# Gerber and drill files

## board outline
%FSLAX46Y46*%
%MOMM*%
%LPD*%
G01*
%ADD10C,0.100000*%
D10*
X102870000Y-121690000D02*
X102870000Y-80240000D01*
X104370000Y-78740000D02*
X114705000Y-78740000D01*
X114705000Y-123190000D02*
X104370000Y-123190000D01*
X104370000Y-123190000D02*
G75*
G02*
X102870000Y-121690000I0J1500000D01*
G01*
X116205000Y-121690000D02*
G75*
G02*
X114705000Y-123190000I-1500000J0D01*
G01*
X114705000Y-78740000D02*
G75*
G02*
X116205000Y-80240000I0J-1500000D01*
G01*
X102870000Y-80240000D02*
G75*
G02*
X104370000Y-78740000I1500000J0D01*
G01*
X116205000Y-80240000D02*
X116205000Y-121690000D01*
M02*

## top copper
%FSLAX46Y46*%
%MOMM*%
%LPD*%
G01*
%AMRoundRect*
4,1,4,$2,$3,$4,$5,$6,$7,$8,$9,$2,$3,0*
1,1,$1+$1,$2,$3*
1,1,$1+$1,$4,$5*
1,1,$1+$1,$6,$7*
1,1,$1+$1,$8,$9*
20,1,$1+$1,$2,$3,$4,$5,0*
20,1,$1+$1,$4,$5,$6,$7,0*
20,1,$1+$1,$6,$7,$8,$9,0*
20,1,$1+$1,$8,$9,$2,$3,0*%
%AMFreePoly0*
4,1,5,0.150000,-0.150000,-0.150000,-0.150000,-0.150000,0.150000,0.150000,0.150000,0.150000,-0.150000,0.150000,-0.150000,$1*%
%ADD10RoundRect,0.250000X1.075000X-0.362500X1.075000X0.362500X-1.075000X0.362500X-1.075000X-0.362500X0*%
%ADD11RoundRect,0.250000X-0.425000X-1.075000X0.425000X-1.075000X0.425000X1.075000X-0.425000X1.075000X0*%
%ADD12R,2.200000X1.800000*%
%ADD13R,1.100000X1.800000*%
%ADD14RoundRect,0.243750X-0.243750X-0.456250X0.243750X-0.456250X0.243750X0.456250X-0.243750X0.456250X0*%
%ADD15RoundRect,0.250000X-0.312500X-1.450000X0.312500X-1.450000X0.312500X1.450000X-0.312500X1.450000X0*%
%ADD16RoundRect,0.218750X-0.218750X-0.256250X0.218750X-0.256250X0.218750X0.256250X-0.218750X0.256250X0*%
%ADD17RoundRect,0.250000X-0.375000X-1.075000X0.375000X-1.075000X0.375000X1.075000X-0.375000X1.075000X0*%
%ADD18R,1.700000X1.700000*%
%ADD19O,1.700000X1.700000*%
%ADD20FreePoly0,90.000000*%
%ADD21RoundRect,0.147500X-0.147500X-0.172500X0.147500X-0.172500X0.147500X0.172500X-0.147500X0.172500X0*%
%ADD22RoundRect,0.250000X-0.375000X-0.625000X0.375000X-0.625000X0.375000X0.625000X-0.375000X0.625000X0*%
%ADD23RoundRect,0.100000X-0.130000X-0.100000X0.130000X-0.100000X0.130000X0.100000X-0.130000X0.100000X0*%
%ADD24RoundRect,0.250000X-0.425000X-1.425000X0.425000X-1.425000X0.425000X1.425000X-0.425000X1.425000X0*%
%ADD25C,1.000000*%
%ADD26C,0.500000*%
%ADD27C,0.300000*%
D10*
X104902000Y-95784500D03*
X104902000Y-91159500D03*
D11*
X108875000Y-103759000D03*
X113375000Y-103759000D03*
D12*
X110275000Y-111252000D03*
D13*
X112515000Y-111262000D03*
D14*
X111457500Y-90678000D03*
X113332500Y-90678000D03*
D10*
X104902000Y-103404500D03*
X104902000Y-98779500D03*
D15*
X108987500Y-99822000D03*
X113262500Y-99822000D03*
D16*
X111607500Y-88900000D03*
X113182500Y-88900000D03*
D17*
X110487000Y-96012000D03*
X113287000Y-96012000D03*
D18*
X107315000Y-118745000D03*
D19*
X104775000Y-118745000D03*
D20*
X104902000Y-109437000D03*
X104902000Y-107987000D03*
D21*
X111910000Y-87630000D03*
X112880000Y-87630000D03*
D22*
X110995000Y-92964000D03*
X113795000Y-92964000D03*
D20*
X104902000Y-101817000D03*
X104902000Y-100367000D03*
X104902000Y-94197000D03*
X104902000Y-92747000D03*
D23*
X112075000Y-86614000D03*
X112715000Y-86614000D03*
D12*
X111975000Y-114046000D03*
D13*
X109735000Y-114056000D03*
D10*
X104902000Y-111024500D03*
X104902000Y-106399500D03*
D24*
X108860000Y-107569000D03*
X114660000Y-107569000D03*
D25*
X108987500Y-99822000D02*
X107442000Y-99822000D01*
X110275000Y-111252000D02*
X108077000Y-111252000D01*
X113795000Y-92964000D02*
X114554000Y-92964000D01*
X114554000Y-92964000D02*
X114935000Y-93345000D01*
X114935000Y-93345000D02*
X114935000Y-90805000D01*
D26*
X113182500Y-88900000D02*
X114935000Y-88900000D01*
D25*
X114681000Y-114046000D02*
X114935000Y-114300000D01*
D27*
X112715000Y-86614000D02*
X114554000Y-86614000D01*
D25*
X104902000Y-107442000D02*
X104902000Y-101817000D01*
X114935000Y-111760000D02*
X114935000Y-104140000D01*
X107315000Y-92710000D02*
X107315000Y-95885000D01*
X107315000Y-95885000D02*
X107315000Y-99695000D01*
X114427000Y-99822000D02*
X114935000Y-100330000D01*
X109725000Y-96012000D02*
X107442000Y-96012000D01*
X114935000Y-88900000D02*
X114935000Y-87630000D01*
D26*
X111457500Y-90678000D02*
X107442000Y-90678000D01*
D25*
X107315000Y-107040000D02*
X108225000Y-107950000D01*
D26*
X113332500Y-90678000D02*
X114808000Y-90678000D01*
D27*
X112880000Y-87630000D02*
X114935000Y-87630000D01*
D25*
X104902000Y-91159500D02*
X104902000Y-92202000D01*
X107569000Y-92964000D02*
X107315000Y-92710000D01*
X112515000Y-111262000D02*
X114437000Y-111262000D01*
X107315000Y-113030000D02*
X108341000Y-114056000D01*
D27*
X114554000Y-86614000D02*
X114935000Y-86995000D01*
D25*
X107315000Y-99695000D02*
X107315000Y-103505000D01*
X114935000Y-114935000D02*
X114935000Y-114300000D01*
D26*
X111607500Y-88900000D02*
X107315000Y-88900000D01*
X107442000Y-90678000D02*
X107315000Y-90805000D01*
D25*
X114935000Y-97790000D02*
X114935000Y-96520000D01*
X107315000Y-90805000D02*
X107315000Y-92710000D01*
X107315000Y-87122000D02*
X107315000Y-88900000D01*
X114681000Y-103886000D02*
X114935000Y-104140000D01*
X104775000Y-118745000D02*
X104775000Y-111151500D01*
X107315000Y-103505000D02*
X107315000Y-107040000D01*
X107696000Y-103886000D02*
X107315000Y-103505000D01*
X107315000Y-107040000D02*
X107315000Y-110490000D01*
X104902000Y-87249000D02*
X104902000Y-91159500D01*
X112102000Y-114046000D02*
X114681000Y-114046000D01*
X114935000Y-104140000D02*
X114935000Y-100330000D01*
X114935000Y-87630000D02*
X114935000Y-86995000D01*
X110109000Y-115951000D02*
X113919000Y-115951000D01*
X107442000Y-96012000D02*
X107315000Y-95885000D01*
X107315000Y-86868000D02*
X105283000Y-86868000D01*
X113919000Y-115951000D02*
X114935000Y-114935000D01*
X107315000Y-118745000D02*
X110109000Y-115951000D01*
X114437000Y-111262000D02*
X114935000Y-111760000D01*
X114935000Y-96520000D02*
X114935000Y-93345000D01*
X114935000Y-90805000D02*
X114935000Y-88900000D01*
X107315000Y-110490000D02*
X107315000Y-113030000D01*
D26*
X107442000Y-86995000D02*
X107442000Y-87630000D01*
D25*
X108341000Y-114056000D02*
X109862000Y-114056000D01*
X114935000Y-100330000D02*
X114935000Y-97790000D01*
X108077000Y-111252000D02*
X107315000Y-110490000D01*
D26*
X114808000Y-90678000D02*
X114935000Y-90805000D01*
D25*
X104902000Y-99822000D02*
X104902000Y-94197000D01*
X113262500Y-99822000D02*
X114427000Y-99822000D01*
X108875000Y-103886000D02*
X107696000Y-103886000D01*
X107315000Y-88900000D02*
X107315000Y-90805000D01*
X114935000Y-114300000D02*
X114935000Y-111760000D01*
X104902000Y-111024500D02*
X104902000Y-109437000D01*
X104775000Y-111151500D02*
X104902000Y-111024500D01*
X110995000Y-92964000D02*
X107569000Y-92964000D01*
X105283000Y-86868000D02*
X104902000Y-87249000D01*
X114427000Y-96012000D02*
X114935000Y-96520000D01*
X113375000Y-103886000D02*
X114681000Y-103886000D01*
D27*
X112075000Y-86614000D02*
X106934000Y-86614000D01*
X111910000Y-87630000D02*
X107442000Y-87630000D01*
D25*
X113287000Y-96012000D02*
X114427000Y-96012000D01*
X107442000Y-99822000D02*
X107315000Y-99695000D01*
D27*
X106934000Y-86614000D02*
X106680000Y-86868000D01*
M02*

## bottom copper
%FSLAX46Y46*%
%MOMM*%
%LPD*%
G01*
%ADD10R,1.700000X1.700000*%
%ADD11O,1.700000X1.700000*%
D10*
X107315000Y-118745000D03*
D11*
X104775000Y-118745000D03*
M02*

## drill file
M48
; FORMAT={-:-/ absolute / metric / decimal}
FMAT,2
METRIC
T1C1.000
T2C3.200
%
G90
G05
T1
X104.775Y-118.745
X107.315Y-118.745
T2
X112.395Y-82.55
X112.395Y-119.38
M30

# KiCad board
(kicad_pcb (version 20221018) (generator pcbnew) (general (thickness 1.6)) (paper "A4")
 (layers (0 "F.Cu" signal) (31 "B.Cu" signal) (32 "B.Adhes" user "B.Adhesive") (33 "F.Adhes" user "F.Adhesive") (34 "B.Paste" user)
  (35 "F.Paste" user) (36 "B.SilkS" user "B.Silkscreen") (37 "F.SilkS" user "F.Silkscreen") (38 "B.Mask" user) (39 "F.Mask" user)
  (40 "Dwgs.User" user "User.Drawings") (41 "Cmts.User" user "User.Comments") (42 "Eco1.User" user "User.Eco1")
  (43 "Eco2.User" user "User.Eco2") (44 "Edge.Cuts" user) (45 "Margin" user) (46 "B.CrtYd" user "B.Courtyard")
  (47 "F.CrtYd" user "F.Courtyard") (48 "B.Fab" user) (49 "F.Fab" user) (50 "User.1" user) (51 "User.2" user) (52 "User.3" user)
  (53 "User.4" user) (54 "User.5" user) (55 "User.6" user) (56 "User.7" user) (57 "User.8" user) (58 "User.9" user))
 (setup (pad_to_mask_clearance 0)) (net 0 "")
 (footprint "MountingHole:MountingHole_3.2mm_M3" (layer "F.Cu") (at 112.395 82.55)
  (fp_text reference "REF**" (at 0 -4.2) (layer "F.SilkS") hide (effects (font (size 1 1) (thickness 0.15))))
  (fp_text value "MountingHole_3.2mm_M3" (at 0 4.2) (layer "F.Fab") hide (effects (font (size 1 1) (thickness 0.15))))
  (pad "" np_thru_hole circle (at 0 0) (size 3.2 3.2) (drill 3.2) (layers "F&B.Cu" "*.Mask")))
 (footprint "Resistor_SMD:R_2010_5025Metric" (layer "F.Cu") (at 104.902 93.472 90)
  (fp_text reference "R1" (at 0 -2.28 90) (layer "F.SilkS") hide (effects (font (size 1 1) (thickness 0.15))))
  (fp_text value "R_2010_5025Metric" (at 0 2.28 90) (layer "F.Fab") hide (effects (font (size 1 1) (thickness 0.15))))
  (pad "1" smd roundrect (at -2.3125 0 90) (size 1.225 2.65) (layers "F.Cu" "F.Paste" "F.Mask") (roundrect_rratio 0.2040816327))
  (pad "2" smd roundrect (at 2.3125 0 90) (size 1.225 2.65) (layers "F.Cu" "F.Paste" "F.Mask") (roundrect_rratio 0.2040816327)))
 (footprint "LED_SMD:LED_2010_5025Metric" (layer "F.Cu") (at 111.125 103.759)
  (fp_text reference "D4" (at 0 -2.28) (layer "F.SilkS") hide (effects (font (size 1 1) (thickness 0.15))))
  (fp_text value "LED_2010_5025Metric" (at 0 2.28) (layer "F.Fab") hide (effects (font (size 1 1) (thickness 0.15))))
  (pad "1" smd roundrect (at -2.25 0) (size 1.35 2.65) (layers "F.Cu" "F.Paste" "F.Mask") (roundrect_rratio 0.1851851852))
  (pad "2" smd roundrect (at 2.25 0) (size 1.35 2.65) (layers "F.Cu" "F.Paste" "F.Mask") (roundrect_rratio 0.1851851852)))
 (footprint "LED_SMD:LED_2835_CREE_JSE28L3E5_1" (layer "F.Cu") (at 111.125 111.252)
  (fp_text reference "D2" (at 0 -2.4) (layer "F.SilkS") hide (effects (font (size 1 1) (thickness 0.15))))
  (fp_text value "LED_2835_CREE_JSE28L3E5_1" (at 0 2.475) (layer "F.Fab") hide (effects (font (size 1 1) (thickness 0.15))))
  (pad "1" smd rect (at -0.85 0) (size 2.2 1.8) (layers "F.Cu" "F.Paste" "F.Mask") (solder_paste_margin -0.18))
  (pad "2" smd rect (at 1.39 0.01) (size 1.1 1.8) (layers "F.Cu" "F.Paste" "F.Mask") (solder_paste_margin -0.18)))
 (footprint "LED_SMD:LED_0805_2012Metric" (layer "F.Cu") (at 112.395 90.678)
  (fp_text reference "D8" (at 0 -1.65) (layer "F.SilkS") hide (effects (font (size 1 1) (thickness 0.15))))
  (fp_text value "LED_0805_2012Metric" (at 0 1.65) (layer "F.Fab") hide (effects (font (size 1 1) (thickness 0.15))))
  (pad "1" smd roundrect (at -0.9375 0) (size 0.975 1.4) (layers "F.Cu" "F.Paste" "F.Mask") (roundrect_rratio 0.25))
  (pad "2" smd roundrect (at 0.9375 0) (size 0.975 1.4) (layers "F.Cu" "F.Paste" "F.Mask") (roundrect_rratio 0.25)))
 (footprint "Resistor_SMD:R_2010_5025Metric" (layer "F.Cu") (at 104.902 101.092 90)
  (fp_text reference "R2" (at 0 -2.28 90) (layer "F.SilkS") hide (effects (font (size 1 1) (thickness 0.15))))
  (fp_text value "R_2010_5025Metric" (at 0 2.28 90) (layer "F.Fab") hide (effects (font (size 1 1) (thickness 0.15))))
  (pad "1" smd roundrect (at -2.3125 0 90) (size 1.225 2.65) (layers "F.Cu" "F.Paste" "F.Mask") (roundrect_rratio 0.2040816327))
  (pad "2" smd roundrect (at 2.3125 0 90) (size 1.225 2.65) (layers "F.Cu" "F.Paste" "F.Mask") (roundrect_rratio 0.2040816327)))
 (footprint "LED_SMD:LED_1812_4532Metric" (layer "F.Cu") (at 111.125 99.822)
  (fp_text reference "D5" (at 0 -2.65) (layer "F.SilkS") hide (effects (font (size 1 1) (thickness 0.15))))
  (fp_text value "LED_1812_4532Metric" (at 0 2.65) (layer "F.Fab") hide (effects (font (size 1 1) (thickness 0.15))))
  (pad "1" smd roundrect (at -2.1375 0) (size 1.125 3.4) (layers "F.Cu" "F.Paste" "F.Mask") (roundrect_rratio 0.2222222222))
  (pad "2" smd roundrect (at 2.1375 0) (size 1.125 3.4) (layers "F.Cu" "F.Paste" "F.Mask") (roundrect_rratio 0.2222222222)))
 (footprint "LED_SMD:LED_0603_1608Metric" (layer "F.Cu") (at 112.395 88.9)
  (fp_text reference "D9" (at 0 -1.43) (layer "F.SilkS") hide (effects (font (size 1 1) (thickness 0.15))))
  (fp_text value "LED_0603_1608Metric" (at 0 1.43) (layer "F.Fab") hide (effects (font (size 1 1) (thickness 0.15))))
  (pad "1" smd roundrect (at -0.7875 0) (size 0.875 0.95) (layers "F.Cu" "F.Paste" "F.Mask") (roundrect_rratio 0.25))
  (pad "2" smd roundrect (at 0.7875 0) (size 0.875 0.95) (layers "F.Cu" "F.Paste" "F.Mask") (roundrect_rratio 0.25)))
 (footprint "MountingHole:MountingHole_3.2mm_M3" (layer "F.Cu") (at 112.395 119.38)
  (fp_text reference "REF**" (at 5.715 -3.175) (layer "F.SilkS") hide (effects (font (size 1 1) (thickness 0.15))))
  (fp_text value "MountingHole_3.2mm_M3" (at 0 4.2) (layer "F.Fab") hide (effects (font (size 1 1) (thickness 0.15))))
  (pad "" np_thru_hole circle (at 0 0) (size 3.2 3.2) (drill 3.2) (layers "*.Cu" "*.Mask")))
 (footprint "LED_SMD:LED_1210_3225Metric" (layer "F.Cu") (at 111.887 96.012)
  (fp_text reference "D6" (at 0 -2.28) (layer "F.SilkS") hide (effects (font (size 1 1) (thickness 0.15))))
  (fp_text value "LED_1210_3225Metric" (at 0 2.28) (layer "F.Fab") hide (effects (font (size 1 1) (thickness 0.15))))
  (pad "1" smd roundrect (at -1.4 0) (size 1.25 2.65) (layers "F.Cu" "F.Paste" "F.Mask") (roundrect_rratio 0.2))
  (pad "2" smd roundrect (at 1.4 0) (size 1.25 2.65) (layers "F.Cu" "F.Paste" "F.Mask") (roundrect_rratio 0.2)))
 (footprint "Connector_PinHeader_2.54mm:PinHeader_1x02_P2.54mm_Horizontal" (layer "F.Cu") (at 107.315 118.745 -90)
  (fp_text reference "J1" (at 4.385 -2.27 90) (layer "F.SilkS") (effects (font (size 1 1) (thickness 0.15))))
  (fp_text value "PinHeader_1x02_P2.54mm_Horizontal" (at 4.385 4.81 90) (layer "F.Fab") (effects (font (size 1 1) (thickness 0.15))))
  (pad "1" thru_hole rect (at 0 0 270) (size 1.7 1.7) (drill 1) (layers "*.Cu" "*.Mask"))
  (pad "2" thru_hole oval (at 0 2.54 270) (size 1.7 1.7) (drill 1) (layers "*.Cu" "*.Mask")))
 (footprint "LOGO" (layer "F.Cu") (at 106.2736 81.9912)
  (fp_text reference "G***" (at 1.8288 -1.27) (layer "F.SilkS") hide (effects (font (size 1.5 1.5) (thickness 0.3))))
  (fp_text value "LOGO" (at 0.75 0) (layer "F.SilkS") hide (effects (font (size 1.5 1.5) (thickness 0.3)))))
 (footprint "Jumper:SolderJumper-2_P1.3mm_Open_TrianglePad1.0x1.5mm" (layer "F.Cu") (at 104.902 108.712 90)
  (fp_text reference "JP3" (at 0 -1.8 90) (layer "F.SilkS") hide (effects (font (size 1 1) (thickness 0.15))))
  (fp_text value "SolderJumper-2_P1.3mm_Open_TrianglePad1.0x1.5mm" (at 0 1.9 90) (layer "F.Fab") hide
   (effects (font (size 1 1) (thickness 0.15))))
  (pad "1" smd custom (at -0.725 0 90) (size 0.3 0.3) (layers "F.Cu" "F.Mask") (zone_connect 2) (options (clearance outline) (anchor rect))
   (primitives))
  (pad "2" smd custom (at 0.725 0 90) (size 0.3 0.3) (layers "F.Cu" "F.Mask") (zone_connect 2) (options (clearance outline) (anchor rect))
   (primitives)))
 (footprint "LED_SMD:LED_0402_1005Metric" (layer "F.Cu") (at 112.395 87.63)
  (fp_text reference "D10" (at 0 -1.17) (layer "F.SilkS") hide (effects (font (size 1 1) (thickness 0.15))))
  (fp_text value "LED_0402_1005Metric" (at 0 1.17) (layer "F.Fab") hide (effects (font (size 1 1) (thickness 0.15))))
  (pad "1" smd roundrect (at -0.485 0) (size 0.59 0.64) (layers "F.Cu" "F.Paste" "F.Mask") (roundrect_rratio 0.25))
  (pad "2" smd roundrect (at 0.485 0) (size 0.59 0.64) (layers "F.Cu" "F.Paste" "F.Mask") (roundrect_rratio 0.25)))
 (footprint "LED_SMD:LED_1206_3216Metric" (layer "F.Cu") (at 112.395 92.964)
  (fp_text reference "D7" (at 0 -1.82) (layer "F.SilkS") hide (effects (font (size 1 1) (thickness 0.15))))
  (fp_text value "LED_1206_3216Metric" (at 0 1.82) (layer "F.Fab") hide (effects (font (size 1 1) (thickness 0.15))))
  (pad "1" smd roundrect (at -1.4 0) (size 1.25 1.75) (layers "F.Cu" "F.Paste" "F.Mask") (roundrect_rratio 0.2))
  (pad "2" smd roundrect (at 1.4 0) (size 1.25 1.75) (layers "F.Cu" "F.Paste" "F.Mask") (roundrect_rratio 0.2)))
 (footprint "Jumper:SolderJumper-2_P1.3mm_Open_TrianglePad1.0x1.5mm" (layer "F.Cu") (at 104.902 101.092 90)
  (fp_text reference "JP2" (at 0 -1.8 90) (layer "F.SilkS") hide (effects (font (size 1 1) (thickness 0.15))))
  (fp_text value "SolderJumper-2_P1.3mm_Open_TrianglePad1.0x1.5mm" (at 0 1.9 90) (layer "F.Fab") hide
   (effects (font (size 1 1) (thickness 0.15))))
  (pad "1" smd custom (at -0.725 0 90) (size 0.3 0.3) (layers "F.Cu" "F.Mask") (zone_connect 2) (options (clearance outline) (anchor rect))
   (primitives))
  (pad "2" smd custom (at 0.725 0 90) (size 0.3 0.3) (layers "F.Cu" "F.Mask") (zone_connect 2) (options (clearance outline) (anchor rect))
   (primitives)))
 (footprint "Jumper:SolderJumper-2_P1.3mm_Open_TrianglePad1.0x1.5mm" (layer "F.Cu") (at 104.902 93.472 90)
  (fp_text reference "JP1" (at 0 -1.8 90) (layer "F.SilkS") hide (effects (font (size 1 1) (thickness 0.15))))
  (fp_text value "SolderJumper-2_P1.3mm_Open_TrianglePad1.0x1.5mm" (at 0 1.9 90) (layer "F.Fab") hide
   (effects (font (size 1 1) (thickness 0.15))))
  (pad "1" smd custom (at -0.725 0 90) (size 0.3 0.3) (layers "F.Cu" "F.Mask") (zone_connect 2) (options (clearance outline) (anchor rect))
   (primitives))
  (pad "2" smd custom (at 0.725 0 90) (size 0.3 0.3) (layers "F.Cu" "F.Mask") (zone_connect 2) (options (clearance outline) (anchor rect))
   (primitives)))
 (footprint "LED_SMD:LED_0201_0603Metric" (layer "F.Cu") (at 112.395 86.614)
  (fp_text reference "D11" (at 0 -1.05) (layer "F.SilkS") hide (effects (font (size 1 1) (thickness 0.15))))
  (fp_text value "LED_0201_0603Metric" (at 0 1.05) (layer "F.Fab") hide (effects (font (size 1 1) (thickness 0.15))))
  (pad "" smd roundrect (at -0.345 0) (size 0.318 0.36) (layers "F.Paste") (roundrect_rratio 0.25))
  (pad "" smd roundrect (at 0.345 0) (size 0.318 0.36) (layers "F.Paste") (roundrect_rratio 0.25))
  (pad "1" smd roundrect (at -0.32 0) (size 0.46 0.4) (layers "F.Cu" "F.Mask") (roundrect_rratio 0.25))
  (pad "2" smd roundrect (at 0.32 0) (size 0.46 0.4) (layers "F.Cu" "F.Mask") (roundrect_rratio 0.25)))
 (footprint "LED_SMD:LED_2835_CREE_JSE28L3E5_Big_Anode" (layer "F.Cu") (at 111.125 114.046)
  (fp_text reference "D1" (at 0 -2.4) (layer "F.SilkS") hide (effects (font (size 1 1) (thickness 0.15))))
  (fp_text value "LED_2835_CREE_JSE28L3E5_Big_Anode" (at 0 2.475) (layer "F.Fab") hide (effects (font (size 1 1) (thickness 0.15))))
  (pad "1" smd rect (at 0.85 0) (size 2.2 1.8) (layers "F.Cu" "F.Paste" "F.Mask") (solder_paste_margin -0.18))
  (pad "2" smd rect (at -1.39 0.01) (size 1.1 1.8) (layers "F.Cu" "F.Paste" "F.Mask") (solder_paste_margin -0.18)))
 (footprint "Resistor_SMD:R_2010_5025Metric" (layer "F.Cu") (at 104.902 108.712 90)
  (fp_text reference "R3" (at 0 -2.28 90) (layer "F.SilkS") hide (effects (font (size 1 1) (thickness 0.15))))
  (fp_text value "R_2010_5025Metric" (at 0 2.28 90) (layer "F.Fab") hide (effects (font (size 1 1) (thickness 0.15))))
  (pad "1" smd roundrect (at -2.3125 0 90) (size 1.225 2.65) (layers "F.Cu" "F.Paste" "F.Mask") (roundrect_rratio 0.2040816327))
  (pad "2" smd roundrect (at 2.3125 0 90) (size 1.225 2.65) (layers "F.Cu" "F.Paste" "F.Mask") (roundrect_rratio 0.2040816327)))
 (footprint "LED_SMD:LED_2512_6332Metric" (layer "F.Cu") (at 111.76 107.569)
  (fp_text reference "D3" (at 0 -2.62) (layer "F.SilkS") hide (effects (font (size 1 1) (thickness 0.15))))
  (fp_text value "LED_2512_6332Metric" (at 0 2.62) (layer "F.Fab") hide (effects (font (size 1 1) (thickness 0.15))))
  (pad "1" smd roundrect (at -2.9 0) (size 1.35 3.35) (layers "F.Cu" "F.Paste" "F.Mask") (roundrect_rratio 0.1851851852))
  (pad "2" smd roundrect (at 2.9 0) (size 1.35 3.35) (layers "F.Cu" "F.Paste" "F.Mask") (roundrect_rratio 0.1851851852)))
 (gr_line (start 102.87 121.69) (end 102.87 80.24) (stroke (width 0.1) (type default)) (layer "Edge.Cuts"))
 (gr_line (start 104.37 78.74) (end 114.705 78.74) (stroke (width 0.1) (type default)) (layer "Edge.Cuts"))
 (gr_line (start 114.705 123.19) (end 104.37 123.19) (stroke (width 0.1) (type default)) (layer "Edge.Cuts"))
 (gr_arc (start 104.37 123.19) (mid 103.30934 122.75066) (end 102.87 121.69) (stroke (width 0.1) (type default)) (layer "Edge.Cuts"))
 (gr_arc (start 116.205 121.69) (mid 115.76566 122.75066) (end 114.705 123.19) (stroke (width 0.1) (type default)) (layer "Edge.Cuts"))
 (gr_arc (start 114.705 78.74) (mid 115.76566 79.17934) (end 116.205 80.24) (stroke (width 0.1) (type default)) (layer "Edge.Cuts"))
 (gr_arc (start 102.87 80.24) (mid 103.30934 79.17934) (end 104.37 78.74) (stroke (width 0.1) (type default)) (layer "Edge.Cuts"))
 (gr_line (start 116.205 80.24) (end 116.205 121.69) (stroke (width 0.1) (type default)) (layer "Edge.Cuts"))
 (segment (start 108.9875 99.822) (end 107.442 99.822) (width 1) (layer "F.Cu") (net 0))
 (segment (start 110.275 111.252) (end 108.077 111.252) (width 1) (layer "F.Cu") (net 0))
 (segment (start 113.795 92.964) (end 114.554 92.964) (width 1) (layer "F.Cu") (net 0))
 (segment (start 114.554 92.964) (end 114.935 93.345) (width 1) (layer "F.Cu") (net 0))
 (segment (start 114.935 93.345) (end 114.935 90.805) (width 1) (layer "F.Cu") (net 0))
 (segment (start 113.1825 88.9) (end 114.935 88.9) (width 0.5) (layer "F.Cu") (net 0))
 (segment (start 114.681 114.046) (end 114.935 114.3) (width 1) (layer "F.Cu") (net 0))
 (segment (start 112.715 86.614) (end 114.554 86.614) (width 0.3) (layer "F.Cu") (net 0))
 (segment (start 104.902 107.442) (end 104.902 101.817) (width 1) (layer "F.Cu") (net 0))
 (segment (start 114.935 111.76) (end 114.935 104.14) (width 1) (layer "F.Cu") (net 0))
 (segment (start 107.315 92.71) (end 107.315 95.885) (width 1) (layer "F.Cu") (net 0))
 (segment (start 107.315 95.885) (end 107.315 99.695) (width 1) (layer "F.Cu") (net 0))
 (segment (start 114.427 99.822) (end 114.935 100.33) (width 1) (layer "F.Cu") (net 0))
 (segment (start 109.725 96.012) (end 107.442 96.012) (width 1) (layer "F.Cu") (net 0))
 (segment (start 114.935 88.9) (end 114.935 87.63) (width 1) (layer "F.Cu") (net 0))
 (segment (start 111.4575 90.678) (end 107.442 90.678) (width 0.5) (layer "F.Cu") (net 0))
 (segment (start 107.315 107.04) (end 108.225 107.95) (width 1) (layer "F.Cu") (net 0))
 (segment (start 113.3325 90.678) (end 114.808 90.678) (width 0.5) (layer "F.Cu") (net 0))
 (segment (start 112.88 87.63) (end 114.935 87.63) (width 0.3) (layer "F.Cu") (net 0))
 (segment (start 104.902 91.1595) (end 104.902 92.202) (width 1) (layer "F.Cu") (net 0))
 (segment (start 107.569 92.964) (end 107.315 92.71) (width 1) (layer "F.Cu") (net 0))
 (segment (start 112.515 111.262) (end 114.437 111.262) (width 1) (layer "F.Cu") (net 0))
 (segment (start 107.315 113.03) (end 108.341 114.056) (width 1) (layer "F.Cu") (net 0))
 (segment (start 114.554 86.614) (end 114.935 86.995) (width 0.3) (layer "F.Cu") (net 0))
 (segment (start 107.315 99.695) (end 107.315 103.505) (width 1) (layer "F.Cu") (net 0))
 (segment (start 114.935 114.935) (end 114.935 114.3) (width 1) (layer "F.Cu") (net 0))
 (segment (start 111.6075 88.9) (end 107.315 88.9) (width 0.5) (layer "F.Cu") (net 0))
 (segment (start 107.442 90.678) (end 107.315 90.805) (width 0.5) (layer "F.Cu") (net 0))
 (segment (start 114.935 97.79) (end 114.935 96.52) (width 1) (layer "F.Cu") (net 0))
 (segment (start 107.315 90.805) (end 107.315 92.71) (width 1) (layer "F.Cu") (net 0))
 (segment (start 107.315 87.122) (end 107.315 88.9) (width 1) (layer "F.Cu") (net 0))
 (segment (start 114.681 103.886) (end 114.935 104.14) (width 1) (layer "F.Cu") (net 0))
 (segment (start 104.775 118.745) (end 104.775 111.1515) (width 1) (layer "F.Cu") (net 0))
 (segment (start 107.315 103.505) (end 107.315 107.04) (width 1) (layer "F.Cu") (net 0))
 (segment (start 107.696 103.886) (end 107.315 103.505) (width 1) (layer "F.Cu") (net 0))
 (segment (start 107.315 107.04) (end 107.315 110.49) (width 1) (layer "F.Cu") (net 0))
 (segment (start 104.902 87.249) (end 104.902 91.1595) (width 1) (layer "F.Cu") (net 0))
 (segment (start 112.102 114.046) (end 114.681 114.046) (width 1) (layer "F.Cu") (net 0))
 (segment (start 114.935 104.14) (end 114.935 100.33) (width 1) (layer "F.Cu") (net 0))
 (segment (start 114.935 87.63) (end 114.935 86.995) (width 1) (layer "F.Cu") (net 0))
 (segment (start 110.109 115.951) (end 113.919 115.951) (width 1) (layer "F.Cu") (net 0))
 (segment (start 107.442 96.012) (end 107.315 95.885) (width 1) (layer "F.Cu") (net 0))
 (segment (start 107.315 86.868) (end 105.283 86.868) (width 1) (layer "F.Cu") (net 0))
 (segment (start 113.919 115.951) (end 114.935 114.935) (width 1) (layer "F.Cu") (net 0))
 (segment (start 107.315 118.745) (end 110.109 115.951) (width 1) (layer "F.Cu") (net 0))
 (segment (start 114.437 111.262) (end 114.935 111.76) (width 1) (layer "F.Cu") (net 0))
 (segment (start 114.935 96.52) (end 114.935 93.345) (width 1) (layer "F.Cu") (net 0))
 (segment (start 114.935 90.805) (end 114.935 88.9) (width 1) (layer "F.Cu") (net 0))
 (segment (start 107.315 110.49) (end 107.315 113.03) (width 1) (layer "F.Cu") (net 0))
 (segment (start 107.442 86.995) (end 107.442 87.63) (width 0.5) (layer "F.Cu") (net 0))
 (segment (start 108.341 114.056) (end 109.862 114.056) (width 1) (layer "F.Cu") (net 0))
 (segment (start 114.935 100.33) (end 114.935 97.79) (width 1) (layer "F.Cu") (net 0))
 (segment (start 108.077 111.252) (end 107.315 110.49) (width 1) (layer "F.Cu") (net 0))
 (segment (start 114.808 90.678) (end 114.935 90.805) (width 0.5) (layer "F.Cu") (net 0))
 (segment (start 104.902 99.822) (end 104.902 94.197) (width 1) (layer "F.Cu") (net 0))
 (segment (start 113.2625 99.822) (end 114.427 99.822) (width 1) (layer "F.Cu") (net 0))
 (segment (start 108.875 103.886) (end 107.696 103.886) (width 1) (layer "F.Cu") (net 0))
 (segment (start 107.315 88.9) (end 107.315 90.805) (width 1) (layer "F.Cu") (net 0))
 (segment (start 114.935 114.3) (end 114.935 111.76) (width 1) (layer "F.Cu") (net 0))
 (segment (start 104.902 111.0245) (end 104.902 109.437) (width 1) (layer "F.Cu") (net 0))
 (segment (start 104.775 111.1515) (end 104.902 111.0245) (width 1) (layer "F.Cu") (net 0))
 (segment (start 110.995 92.964) (end 107.569 92.964) (width 1) (layer "F.Cu") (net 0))
 (segment (start 105.283 86.868) (end 104.902 87.249) (width 1) (layer "F.Cu") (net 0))
 (segment (start 114.427 96.012) (end 114.935 96.52) (width 1) (layer "F.Cu") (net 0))
 (segment (start 113.375 103.886) (end 114.681 103.886) (width 1) (layer "F.Cu") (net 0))
 (segment (start 112.075 86.614) (end 106.934 86.614) (width 0.3) (layer "F.Cu") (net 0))
 (segment (start 111.91 87.63) (end 107.442 87.63) (width 0.3) (layer "F.Cu") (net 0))
 (segment (start 113.287 96.012) (end 114.427 96.012) (width 1) (layer "F.Cu") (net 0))
 (segment (start 107.442 99.822) (end 107.315 99.695) (width 1) (layer "F.Cu") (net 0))
 (segment (start 106.934 86.614) (end 106.68 86.868) (width 0.3) (layer "F.Cu") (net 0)))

